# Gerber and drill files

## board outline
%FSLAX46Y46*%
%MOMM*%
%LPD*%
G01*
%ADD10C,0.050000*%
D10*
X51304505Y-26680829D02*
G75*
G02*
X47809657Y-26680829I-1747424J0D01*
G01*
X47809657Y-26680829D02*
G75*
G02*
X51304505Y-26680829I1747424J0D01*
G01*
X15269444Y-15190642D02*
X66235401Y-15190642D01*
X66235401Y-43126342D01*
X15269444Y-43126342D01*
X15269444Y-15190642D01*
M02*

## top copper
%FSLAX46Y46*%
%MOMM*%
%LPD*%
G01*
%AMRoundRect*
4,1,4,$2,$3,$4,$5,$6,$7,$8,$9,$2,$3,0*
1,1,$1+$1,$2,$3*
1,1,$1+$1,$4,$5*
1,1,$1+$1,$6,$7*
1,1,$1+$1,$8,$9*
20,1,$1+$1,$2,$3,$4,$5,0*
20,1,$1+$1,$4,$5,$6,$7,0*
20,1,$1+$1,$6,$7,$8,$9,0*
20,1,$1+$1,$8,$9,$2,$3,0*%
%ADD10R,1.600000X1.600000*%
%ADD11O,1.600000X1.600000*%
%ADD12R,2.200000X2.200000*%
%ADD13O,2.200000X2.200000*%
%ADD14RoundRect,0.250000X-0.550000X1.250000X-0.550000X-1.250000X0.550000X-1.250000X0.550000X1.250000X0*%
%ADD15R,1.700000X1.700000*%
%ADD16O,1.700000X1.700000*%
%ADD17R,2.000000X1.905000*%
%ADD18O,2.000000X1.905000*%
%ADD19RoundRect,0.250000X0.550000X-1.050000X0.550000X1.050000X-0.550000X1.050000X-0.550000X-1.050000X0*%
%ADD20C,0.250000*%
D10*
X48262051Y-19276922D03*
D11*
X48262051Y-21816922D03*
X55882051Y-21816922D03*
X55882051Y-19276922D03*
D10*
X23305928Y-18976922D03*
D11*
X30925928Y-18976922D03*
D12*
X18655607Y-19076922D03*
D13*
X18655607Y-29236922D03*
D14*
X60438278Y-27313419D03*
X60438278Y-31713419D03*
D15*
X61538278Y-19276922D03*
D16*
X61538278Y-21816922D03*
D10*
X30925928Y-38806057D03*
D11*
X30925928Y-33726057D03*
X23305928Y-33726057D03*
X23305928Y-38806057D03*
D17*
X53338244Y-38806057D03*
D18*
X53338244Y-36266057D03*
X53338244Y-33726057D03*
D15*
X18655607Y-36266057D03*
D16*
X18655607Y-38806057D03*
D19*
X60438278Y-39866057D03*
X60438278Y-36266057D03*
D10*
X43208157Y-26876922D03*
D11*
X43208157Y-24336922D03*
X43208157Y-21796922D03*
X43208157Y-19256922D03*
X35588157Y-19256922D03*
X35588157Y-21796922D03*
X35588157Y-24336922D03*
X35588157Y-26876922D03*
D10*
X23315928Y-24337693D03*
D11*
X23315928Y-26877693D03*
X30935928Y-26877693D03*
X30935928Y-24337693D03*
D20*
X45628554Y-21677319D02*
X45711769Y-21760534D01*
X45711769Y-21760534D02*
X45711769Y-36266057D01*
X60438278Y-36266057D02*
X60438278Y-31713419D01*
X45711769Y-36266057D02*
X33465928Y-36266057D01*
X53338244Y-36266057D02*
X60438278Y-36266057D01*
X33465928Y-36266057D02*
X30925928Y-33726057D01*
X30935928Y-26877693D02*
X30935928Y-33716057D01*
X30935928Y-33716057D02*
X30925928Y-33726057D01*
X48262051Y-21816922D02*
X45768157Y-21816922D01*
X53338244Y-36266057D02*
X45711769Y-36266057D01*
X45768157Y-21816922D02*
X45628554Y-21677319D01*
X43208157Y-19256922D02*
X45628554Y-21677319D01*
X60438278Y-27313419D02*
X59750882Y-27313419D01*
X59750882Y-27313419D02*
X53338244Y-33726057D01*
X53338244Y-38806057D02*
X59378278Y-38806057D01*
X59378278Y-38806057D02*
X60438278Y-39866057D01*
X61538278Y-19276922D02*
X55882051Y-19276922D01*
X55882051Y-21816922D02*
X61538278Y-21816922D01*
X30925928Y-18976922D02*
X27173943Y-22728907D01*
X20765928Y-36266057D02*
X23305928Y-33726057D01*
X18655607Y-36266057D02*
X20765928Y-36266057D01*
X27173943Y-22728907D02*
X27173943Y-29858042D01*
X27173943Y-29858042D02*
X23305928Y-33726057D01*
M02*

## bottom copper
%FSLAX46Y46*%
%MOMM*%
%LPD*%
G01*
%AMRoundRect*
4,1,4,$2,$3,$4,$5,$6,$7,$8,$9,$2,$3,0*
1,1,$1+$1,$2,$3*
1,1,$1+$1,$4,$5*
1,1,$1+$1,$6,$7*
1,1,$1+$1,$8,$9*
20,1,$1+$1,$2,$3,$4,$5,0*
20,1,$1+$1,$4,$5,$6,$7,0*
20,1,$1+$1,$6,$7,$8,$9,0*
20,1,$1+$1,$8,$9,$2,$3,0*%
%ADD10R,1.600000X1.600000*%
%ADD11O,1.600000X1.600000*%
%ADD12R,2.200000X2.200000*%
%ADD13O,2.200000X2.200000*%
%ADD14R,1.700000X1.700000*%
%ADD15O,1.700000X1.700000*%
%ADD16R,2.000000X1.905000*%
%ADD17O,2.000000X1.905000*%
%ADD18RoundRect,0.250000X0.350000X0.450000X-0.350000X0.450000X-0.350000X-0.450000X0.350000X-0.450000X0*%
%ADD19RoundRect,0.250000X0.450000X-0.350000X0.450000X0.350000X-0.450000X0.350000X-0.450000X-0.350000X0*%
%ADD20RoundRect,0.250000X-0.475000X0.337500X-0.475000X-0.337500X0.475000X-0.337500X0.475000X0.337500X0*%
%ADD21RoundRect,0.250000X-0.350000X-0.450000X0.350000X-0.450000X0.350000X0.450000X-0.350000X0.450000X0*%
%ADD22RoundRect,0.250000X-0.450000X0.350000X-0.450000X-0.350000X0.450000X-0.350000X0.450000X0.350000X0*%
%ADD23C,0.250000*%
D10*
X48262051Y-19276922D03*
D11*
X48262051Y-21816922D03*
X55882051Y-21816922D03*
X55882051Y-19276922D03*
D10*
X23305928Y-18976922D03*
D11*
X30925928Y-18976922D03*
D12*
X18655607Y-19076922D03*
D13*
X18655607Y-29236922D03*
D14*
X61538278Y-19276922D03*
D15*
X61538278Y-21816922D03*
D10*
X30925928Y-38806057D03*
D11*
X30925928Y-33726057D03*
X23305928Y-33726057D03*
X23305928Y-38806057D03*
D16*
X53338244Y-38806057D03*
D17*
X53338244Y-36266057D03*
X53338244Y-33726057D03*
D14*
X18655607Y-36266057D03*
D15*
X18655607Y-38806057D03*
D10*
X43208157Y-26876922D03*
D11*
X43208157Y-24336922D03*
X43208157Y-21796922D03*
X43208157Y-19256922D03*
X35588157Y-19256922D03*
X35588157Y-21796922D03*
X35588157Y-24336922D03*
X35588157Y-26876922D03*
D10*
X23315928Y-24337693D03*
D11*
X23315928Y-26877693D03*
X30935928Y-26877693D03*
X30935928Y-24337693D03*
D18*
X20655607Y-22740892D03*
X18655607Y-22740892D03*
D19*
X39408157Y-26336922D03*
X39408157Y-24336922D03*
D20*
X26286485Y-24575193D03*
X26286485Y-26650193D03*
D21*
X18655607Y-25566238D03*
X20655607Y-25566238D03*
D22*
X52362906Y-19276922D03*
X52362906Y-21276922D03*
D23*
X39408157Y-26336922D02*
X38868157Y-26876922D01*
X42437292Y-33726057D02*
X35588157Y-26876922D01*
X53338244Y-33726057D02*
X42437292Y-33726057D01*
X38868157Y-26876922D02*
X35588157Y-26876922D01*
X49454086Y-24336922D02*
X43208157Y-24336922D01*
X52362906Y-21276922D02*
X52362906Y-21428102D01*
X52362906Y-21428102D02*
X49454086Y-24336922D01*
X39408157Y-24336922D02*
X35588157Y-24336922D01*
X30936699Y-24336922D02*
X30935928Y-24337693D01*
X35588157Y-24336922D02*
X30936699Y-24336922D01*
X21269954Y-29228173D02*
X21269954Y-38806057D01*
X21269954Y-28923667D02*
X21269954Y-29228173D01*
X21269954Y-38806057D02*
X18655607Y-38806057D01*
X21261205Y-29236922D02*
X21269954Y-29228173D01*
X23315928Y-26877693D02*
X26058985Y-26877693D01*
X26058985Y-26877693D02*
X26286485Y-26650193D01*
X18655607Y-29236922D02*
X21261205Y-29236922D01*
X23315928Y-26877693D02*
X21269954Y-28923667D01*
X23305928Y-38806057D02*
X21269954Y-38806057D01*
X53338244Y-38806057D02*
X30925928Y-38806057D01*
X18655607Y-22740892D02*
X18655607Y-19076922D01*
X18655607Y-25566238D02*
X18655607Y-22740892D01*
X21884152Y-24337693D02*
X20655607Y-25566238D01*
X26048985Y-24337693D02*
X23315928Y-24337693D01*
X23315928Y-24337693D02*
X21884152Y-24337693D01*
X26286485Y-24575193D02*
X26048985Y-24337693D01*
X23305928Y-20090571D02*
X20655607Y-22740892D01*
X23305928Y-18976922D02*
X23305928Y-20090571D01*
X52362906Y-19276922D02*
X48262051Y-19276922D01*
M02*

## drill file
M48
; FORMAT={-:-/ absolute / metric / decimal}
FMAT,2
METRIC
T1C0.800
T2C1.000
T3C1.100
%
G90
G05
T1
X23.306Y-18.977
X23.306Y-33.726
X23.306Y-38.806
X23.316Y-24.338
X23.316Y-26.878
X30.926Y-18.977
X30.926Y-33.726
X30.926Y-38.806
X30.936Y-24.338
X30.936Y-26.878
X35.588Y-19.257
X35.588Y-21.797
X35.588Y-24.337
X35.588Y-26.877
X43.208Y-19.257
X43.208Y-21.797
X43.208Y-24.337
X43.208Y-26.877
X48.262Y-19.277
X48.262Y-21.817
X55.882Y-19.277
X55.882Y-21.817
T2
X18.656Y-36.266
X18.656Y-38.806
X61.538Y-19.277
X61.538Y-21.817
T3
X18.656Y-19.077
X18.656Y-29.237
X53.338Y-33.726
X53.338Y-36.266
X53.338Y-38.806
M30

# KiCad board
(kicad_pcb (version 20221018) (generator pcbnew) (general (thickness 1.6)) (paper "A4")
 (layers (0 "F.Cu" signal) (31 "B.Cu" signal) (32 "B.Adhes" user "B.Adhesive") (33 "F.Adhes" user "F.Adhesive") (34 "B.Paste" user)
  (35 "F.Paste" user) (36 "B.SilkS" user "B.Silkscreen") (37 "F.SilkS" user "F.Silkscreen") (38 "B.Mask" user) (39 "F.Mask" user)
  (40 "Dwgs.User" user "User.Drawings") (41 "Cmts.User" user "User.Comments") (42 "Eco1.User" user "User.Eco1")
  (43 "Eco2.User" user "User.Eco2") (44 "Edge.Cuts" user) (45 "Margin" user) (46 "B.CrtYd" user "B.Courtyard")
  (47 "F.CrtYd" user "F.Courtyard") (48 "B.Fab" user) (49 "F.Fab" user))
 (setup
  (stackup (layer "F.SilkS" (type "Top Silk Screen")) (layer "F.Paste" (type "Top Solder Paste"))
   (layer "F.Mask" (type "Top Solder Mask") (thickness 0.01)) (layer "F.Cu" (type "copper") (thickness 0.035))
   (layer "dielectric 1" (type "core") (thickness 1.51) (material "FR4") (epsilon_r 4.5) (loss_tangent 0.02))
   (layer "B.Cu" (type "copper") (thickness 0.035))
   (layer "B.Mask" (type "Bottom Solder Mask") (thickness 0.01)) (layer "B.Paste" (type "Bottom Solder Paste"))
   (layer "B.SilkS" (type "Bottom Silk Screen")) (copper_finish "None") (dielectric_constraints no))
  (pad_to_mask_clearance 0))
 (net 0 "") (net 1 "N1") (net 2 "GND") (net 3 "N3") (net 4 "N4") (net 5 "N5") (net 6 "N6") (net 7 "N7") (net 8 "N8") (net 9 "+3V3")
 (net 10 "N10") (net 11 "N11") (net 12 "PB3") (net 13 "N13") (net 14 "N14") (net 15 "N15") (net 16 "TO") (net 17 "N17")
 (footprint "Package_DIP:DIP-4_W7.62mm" (layer "F.Cu") (at 48.262051 19.276922)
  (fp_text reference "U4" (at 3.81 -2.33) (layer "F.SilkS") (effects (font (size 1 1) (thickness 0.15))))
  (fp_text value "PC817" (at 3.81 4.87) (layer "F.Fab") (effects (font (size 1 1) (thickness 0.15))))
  (pad "1" thru_hole rect (at 0 0) (size 1.6 1.6) (drill 0.8) (layers "*.Cu" "*.Mask") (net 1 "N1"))
  (pad "2" thru_hole oval (at 0 2.54) (size 1.6 1.6) (drill 0.8) (layers "*.Cu" "*.Mask") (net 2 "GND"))
  (pad "3" thru_hole oval (at 7.62 2.54) (size 1.6 1.6) (drill 0.8) (layers "*.Cu" "*.Mask") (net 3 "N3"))
  (pad "4" thru_hole oval (at 7.62 0) (size 1.6 1.6) (drill 0.8) (layers "*.Cu" "*.Mask") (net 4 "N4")))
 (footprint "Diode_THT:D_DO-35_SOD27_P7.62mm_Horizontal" (layer "F.Cu") (at 23.305928 18.976922)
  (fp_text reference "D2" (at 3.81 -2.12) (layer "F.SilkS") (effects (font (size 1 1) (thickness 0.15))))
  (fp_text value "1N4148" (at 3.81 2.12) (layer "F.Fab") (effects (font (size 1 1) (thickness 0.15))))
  (pad "1" thru_hole rect (at 0 0) (size 1.6 1.6) (drill 0.8) (layers "*.Cu" "*.Mask") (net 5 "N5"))
  (pad "2" thru_hole oval (at 7.62 0) (size 1.6 1.6) (drill 0.8) (layers "*.Cu" "*.Mask") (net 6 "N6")))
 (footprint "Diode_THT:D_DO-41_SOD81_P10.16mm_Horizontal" (layer "F.Cu") (at 18.655607 19.076922 -90)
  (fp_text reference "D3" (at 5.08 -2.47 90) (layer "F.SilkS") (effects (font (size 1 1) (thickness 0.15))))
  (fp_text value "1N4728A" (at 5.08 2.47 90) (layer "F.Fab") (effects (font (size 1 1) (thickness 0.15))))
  (pad "1" thru_hole rect (at 0 0 270) (size 2.2 2.2) (drill 1.1) (layers "*.Cu" "*.Mask") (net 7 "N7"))
  (pad "2" thru_hole oval (at 10.16 0 270) (size 2.2 2.2) (drill 1.1) (layers "*.Cu" "*.Mask") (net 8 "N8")))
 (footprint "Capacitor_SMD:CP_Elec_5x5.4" (layer "F.Cu") (at 60.438278 29.513419 -90)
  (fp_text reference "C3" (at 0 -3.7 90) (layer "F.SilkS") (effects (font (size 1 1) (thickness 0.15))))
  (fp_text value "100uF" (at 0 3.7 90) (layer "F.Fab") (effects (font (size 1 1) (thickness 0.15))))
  (pad "1" smd roundrect (at -2.2 0 270) (size 3 1.6) (layers "F.Cu" "F.Paste" "F.Mask") (roundrect_rratio 0.15625) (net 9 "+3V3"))
  (pad "2" smd roundrect (at 2.2 0 270) (size 3 1.6) (layers "F.Cu" "F.Paste" "F.Mask") (roundrect_rratio 0.15625) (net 2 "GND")))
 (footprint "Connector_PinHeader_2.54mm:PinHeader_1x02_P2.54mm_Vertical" (layer "F.Cu") (at 61.538278 19.276922)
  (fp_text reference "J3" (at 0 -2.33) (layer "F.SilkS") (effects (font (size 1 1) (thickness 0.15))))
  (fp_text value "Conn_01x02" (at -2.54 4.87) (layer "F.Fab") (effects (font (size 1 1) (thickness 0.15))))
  (pad "1" thru_hole rect (at 0 0) (size 1.7 1.7) (drill 1) (layers "*.Cu" "*.Mask") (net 4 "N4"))
  (pad "2" thru_hole oval (at 0 2.54) (size 1.7 1.7) (drill 1) (layers "*.Cu" "*.Mask") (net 3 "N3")))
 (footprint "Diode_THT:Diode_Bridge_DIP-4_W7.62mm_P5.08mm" (layer "F.Cu") (at 30.925928 38.806057 180)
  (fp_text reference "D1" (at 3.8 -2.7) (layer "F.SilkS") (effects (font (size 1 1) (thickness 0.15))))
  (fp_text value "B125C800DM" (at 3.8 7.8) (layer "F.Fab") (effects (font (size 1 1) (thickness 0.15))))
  (pad "1" thru_hole rect (at 0 0 180) (size 1.6 1.6) (drill 0.8) (layers "*.Cu" "*.Mask") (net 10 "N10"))
  (pad "2" thru_hole oval (at 0 5.08 180) (size 1.6 1.6) (drill 0.8) (layers "*.Cu" "*.Mask") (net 2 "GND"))
  (pad "3" thru_hole oval (at 7.62 5.08 180) (size 1.6 1.6) (drill 0.8) (layers "*.Cu" "*.Mask") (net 6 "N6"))
  (pad "4" thru_hole oval (at 7.62 0 180) (size 1.6 1.6) (drill 0.8) (layers "*.Cu" "*.Mask") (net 8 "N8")))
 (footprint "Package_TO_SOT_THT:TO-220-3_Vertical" (layer "F.Cu") (at 53.338244 38.806057 90)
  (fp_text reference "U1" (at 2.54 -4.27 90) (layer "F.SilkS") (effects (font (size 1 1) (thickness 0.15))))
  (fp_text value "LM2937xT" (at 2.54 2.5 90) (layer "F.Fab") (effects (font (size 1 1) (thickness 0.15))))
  (pad "1" thru_hole rect (at 0 0 90) (size 1.905 2) (drill 1.1) (layers "*.Cu" "*.Mask") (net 10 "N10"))
  (pad "2" thru_hole oval (at 2.54 0 90) (size 1.905 2) (drill 1.1) (layers "*.Cu" "*.Mask") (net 2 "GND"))
  (pad "3" thru_hole oval (at 5.08 0 90) (size 1.905 2) (drill 1.1) (layers "*.Cu" "*.Mask") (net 9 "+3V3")))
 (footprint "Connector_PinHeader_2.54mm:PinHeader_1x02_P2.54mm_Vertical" (layer "F.Cu") (at 18.655607 36.266057)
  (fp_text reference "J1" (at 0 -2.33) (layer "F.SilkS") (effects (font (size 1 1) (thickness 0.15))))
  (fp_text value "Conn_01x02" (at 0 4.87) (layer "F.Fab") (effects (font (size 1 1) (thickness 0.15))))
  (pad "1" thru_hole rect (at 0 0) (size 1.7 1.7) (drill 1) (layers "*.Cu" "*.Mask") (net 6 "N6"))
  (pad "2" thru_hole oval (at 0 2.54) (size 1.7 1.7) (drill 1) (layers "*.Cu" "*.Mask") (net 8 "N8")))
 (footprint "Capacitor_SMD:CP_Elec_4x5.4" (layer "F.Cu") (at 60.438278 38.066057 90)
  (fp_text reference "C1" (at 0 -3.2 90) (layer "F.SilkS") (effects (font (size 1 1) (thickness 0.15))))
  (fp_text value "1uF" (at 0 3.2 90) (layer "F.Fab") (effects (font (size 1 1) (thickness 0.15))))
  (pad "1" smd roundrect (at -1.8 0 90) (size 2.6 1.6) (layers "F.Cu" "F.Paste" "F.Mask") (roundrect_rratio 0.15625) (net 10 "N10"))
  (pad "2" smd roundrect (at 1.8 0 90) (size 2.6 1.6) (layers "F.Cu" "F.Paste" "F.Mask") (roundrect_rratio 0.15625) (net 2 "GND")))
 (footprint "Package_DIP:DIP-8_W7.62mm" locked (layer "F.Cu") (at 43.208157 26.876922 180)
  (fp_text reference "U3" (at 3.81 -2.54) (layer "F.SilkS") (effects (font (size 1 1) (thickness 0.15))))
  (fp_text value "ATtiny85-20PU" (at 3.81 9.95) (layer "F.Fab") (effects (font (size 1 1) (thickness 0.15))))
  (pad "1" thru_hole rect locked (at 0 0 180) (size 1.6 1.6) (drill 0.8) (layers "*.Cu" "*.Mask") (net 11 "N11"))
  (pad "2" thru_hole oval locked (at 0 2.54 180) (size 1.6 1.6) (drill 0.8) (layers "*.Cu" "*.Mask") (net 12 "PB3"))
  (pad "3" thru_hole oval locked (at 0 5.08 180) (size 1.6 1.6) (drill 0.8) (layers "*.Cu" "*.Mask") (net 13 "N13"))
  (pad "4" thru_hole oval locked (at 0 7.62 180) (size 1.6 1.6) (drill 0.8) (layers "*.Cu" "*.Mask") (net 2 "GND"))
  (pad "5" thru_hole oval locked (at 7.62 7.62 180) (size 1.6 1.6) (drill 0.8) (layers "*.Cu" "*.Mask") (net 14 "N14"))
  (pad "6" thru_hole oval locked (at 7.62 5.08 180) (size 1.6 1.6) (drill 0.8) (layers "*.Cu" "*.Mask") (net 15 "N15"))
  (pad "7" thru_hole oval locked (at 7.62 2.54 180) (size 1.6 1.6) (drill 0.8) (layers "*.Cu" "*.Mask") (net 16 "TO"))
  (pad "8" thru_hole oval locked (at 7.62 0 180) (size 1.6 1.6) (drill 0.8) (layers "*.Cu" "*.Mask") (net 9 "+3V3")))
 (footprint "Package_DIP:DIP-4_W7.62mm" (layer "F.Cu") (at 23.315928 24.337693)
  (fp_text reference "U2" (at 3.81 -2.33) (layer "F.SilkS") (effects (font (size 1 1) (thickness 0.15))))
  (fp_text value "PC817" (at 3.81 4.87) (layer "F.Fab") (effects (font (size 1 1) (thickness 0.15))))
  (pad "1" thru_hole rect (at 0 0) (size 1.6 1.6) (drill 0.8) (layers "*.Cu" "*.Mask") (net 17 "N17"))
  (pad "2" thru_hole oval (at 0 2.54) (size 1.6 1.6) (drill 0.8) (layers "*.Cu" "*.Mask") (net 8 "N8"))
  (pad "3" thru_hole oval (at 7.62 2.54) (size 1.6 1.6) (drill 0.8) (layers "*.Cu" "*.Mask") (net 2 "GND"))
  (pad "4" thru_hole oval (at 7.62 0) (size 1.6 1.6) (drill 0.8) (layers "*.Cu" "*.Mask") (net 16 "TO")))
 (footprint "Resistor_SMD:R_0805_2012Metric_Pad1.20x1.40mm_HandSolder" (layer "B.Cu") (at 19.655607 22.740892 180)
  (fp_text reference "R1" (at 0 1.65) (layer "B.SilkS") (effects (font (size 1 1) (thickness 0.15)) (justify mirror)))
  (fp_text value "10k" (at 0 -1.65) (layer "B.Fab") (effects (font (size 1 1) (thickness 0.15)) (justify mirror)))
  (pad "1" smd roundrect (at -1 0 180) (size 1.2 1.4) (layers "B.Cu" "B.Paste" "B.Mask") (roundrect_rratio 0.208333) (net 5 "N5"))
  (pad "2" smd roundrect (at 1 0 180) (size 1.2 1.4) (layers "B.Cu" "B.Paste" "B.Mask") (roundrect_rratio 0.208333) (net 7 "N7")))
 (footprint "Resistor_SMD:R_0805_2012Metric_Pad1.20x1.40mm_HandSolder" (layer "B.Cu") (at 39.408157 25.336922 90)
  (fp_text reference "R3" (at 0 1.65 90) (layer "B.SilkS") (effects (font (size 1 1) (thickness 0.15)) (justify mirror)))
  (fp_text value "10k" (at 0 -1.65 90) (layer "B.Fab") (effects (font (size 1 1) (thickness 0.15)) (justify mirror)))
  (pad "1" smd roundrect (at -1 0 90) (size 1.2 1.4) (layers "B.Cu" "B.Paste" "B.Mask") (roundrect_rratio 0.208333) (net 9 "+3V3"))
  (pad "2" smd roundrect (at 1 0 90) (size 1.2 1.4) (layers "B.Cu" "B.Paste" "B.Mask") (roundrect_rratio 0.208333) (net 16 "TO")))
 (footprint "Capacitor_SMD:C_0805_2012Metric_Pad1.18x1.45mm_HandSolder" (layer "B.Cu") (at 26.286485 25.612693 -90)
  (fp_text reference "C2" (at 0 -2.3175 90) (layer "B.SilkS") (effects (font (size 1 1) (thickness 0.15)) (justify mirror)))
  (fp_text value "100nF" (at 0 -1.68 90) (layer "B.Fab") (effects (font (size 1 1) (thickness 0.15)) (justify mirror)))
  (pad "1" smd roundrect (at -1.0375 0 270) (size 1.175 1.45) (layers "B.Cu" "B.Paste" "B.Mask") (roundrect_rratio 0.212766) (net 17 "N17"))
  (pad "2" smd roundrect (at 1.0375 0 270) (size 1.175 1.45) (layers "B.Cu" "B.Paste" "B.Mask") (roundrect_rratio 0.212766) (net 8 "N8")))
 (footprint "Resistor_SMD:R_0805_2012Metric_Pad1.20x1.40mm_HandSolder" (layer "B.Cu") (at 19.655607 25.566238)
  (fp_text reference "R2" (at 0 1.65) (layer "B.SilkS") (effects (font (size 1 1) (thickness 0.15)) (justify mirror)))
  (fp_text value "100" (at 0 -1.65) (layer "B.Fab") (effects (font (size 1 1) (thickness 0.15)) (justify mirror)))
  (pad "1" smd roundrect (at -1 0) (size 1.2 1.4) (layers "B.Cu" "B.Paste" "B.Mask") (roundrect_rratio 0.208333) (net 7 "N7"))
  (pad "2" smd roundrect (at 1 0) (size 1.2 1.4) (layers "B.Cu" "B.Paste" "B.Mask") (roundrect_rratio 0.208333) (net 17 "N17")))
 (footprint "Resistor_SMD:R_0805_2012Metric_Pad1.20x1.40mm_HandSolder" (layer "B.Cu") (at 52.362906 20.276922 -90)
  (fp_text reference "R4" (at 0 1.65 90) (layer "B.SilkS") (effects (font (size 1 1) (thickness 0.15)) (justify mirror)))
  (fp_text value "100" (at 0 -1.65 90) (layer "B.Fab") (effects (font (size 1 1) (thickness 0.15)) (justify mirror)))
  (pad "1" smd roundrect (at -1 0 270) (size 1.2 1.4) (layers "B.Cu" "B.Paste" "B.Mask") (roundrect_rratio 0.208333) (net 1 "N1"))
  (pad "2" smd roundrect (at 1 0 270) (size 1.2 1.4) (layers "B.Cu" "B.Paste" "B.Mask") (roundrect_rratio 0.208333) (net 12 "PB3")))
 (gr_circle (center 49.557081 26.680829) (end 50.875697 27.827451) (stroke (width 0.05) (type default)) (fill none) (layer "Edge.Cuts"))
 (gr_rect (start 15.269444 15.190642) (end 66.235401 43.126342) (stroke (width 0.05) (type default)) (fill none) (layer "Edge.Cuts"))
 (segment (start 45.628554 21.677319) (end 45.711769 21.760534) (width 0.25) (layer "F.Cu") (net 2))
 (segment (start 45.711769 21.760534) (end 45.711769 36.266057) (width 0.25) (layer "F.Cu") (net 2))
 (segment (start 60.438278 36.266057) (end 60.438278 31.713419) (width 0.25) (layer "F.Cu") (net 2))
 (segment (start 45.711769 36.266057) (end 33.465928 36.266057) (width 0.25) (layer "F.Cu") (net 2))
 (segment (start 53.338244 36.266057) (end 60.438278 36.266057) (width 0.25) (layer "F.Cu") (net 2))
 (segment (start 33.465928 36.266057) (end 30.925928 33.726057) (width 0.25) (layer "F.Cu") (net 2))
 (segment (start 30.935928 26.877693) (end 30.935928 33.716057) (width 0.25) (layer "F.Cu") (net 2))
 (segment (start 30.935928 33.716057) (end 30.925928 33.726057) (width 0.25) (layer "F.Cu") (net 2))
 (segment (start 48.262051 21.816922) (end 45.768157 21.816922) (width 0.25) (layer "F.Cu") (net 2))
 (segment (start 53.338244 36.266057) (end 45.711769 36.266057) (width 0.25) (layer "F.Cu") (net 2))
 (segment (start 45.768157 21.816922) (end 45.628554 21.677319) (width 0.25) (layer "F.Cu") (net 2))
 (segment (start 43.208157 19.256922) (end 45.628554 21.677319) (width 0.25) (layer "F.Cu") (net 2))
 (segment (start 60.438278 27.313419) (end 59.750882 27.313419) (width 0.25) (layer "F.Cu") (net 9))
 (segment (start 59.750882 27.313419) (end 53.338244 33.726057) (width 0.25) (layer "F.Cu") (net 9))
 (segment (start 39.408157 26.336922) (end 38.868157 26.876922) (width 0.25) (layer "B.Cu") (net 9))
 (segment (start 42.437292 33.726057) (end 35.588157 26.876922) (width 0.25) (layer "B.Cu") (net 9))
 (segment (start 53.338244 33.726057) (end 42.437292 33.726057) (width 0.25) (layer "B.Cu") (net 9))
 (segment (start 38.868157 26.876922) (end 35.588157 26.876922) (width 0.25) (layer "B.Cu") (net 9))
 (segment (start 49.454086 24.336922) (end 43.208157 24.336922) (width 0.25) (layer "B.Cu") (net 12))
 (segment (start 52.362906 21.276922) (end 52.362906 21.428102) (width 0.25) (layer "B.Cu") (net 12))
 (segment (start 52.362906 21.428102) (end 49.454086 24.336922) (width 0.25) (layer "B.Cu") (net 12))
 (segment (start 39.408157 24.336922) (end 35.588157 24.336922) (width 0.25) (layer "B.Cu") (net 16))
 (segment (start 30.936699 24.336922) (end 30.935928 24.337693) (width 0.25) (layer "B.Cu") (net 16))
 (segment (start 35.588157 24.336922) (end 30.936699 24.336922) (width 0.25) (layer "B.Cu") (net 16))
 (segment (start 21.269954 29.228173) (end 21.269954 38.806057) (width 0.25) (layer "B.Cu") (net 8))
 (segment (start 21.269954 28.923667) (end 21.269954 29.228173) (width 0.25) (layer "B.Cu") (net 8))
 (segment (start 21.269954 38.806057) (end 18.655607 38.806057) (width 0.25) (layer "B.Cu") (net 8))
 (segment (start 21.261205 29.236922) (end 21.269954 29.228173) (width 0.25) (layer "B.Cu") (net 8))
 (segment (start 23.315928 26.877693) (end 26.058985 26.877693) (width 0.25) (layer "B.Cu") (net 8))
 (segment (start 26.058985 26.877693) (end 26.286485 26.650193) (width 0.25) (layer "B.Cu") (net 8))
 (segment (start 18.655607 29.236922) (end 21.261205 29.236922) (width 0.25) (layer "B.Cu") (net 8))
 (segment (start 23.315928 26.877693) (end 21.269954 28.923667) (width 0.25) (layer "B.Cu") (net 8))
 (segment (start 23.305928 38.806057) (end 21.269954 38.806057) (width 0.25) (layer "B.Cu") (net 8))
 (segment (start 53.338244 38.806057) (end 59.378278 38.806057) (width 0.25) (layer "F.Cu") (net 10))
 (segment (start 59.378278 38.806057) (end 60.438278 39.866057) (width 0.25) (layer "F.Cu") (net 10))
 (segment (start 53.338244 38.806057) (end 30.925928 38.806057) (width 0.25) (layer "B.Cu") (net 10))
 (segment (start 18.655607 22.740892) (end 18.655607 19.076922) (width 0.25) (layer "B.Cu") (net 7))
 (segment (start 18.655607 25.566238) (end 18.655607 22.740892) (width 0.25) (layer "B.Cu") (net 7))
 (segment (start 61.538278 19.276922) (end 55.882051 19.276922) (width 0.25) (layer "F.Cu") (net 4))
 (segment (start 55.882051 21.816922) (end 61.538278 21.816922) (width 0.25) (layer "F.Cu") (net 3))
 (segment (start 21.884152 24.337693) (end 20.655607 25.566238) (width 0.25) (layer "B.Cu") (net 17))
 (segment (start 26.048985 24.337693) (end 23.315928 24.337693) (width 0.25) (layer "B.Cu") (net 17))
 (segment (start 23.315928 24.337693) (end 21.884152 24.337693) (width 0.25) (layer "B.Cu") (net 17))
 (segment (start 26.286485 24.575193) (end 26.048985 24.337693) (width 0.25) (layer "B.Cu") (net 17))
 (segment (start 30.925928 18.976922) (end 27.173943 22.728907) (width 0.25) (layer "F.Cu") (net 6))
 (segment (start 20.765928 36.266057) (end 23.305928 33.726057) (width 0.25) (layer "F.Cu") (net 6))
 (segment (start 18.655607 36.266057) (end 20.765928 36.266057) (width 0.25) (layer "F.Cu") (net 6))
 (segment (start 27.173943 22.728907) (end 27.173943 29.858042) (width 0.25) (layer "F.Cu") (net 6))
 (segment (start 27.173943 29.858042) (end 23.305928 33.726057) (width 0.25) (layer "F.Cu") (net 6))
 (segment (start 23.305928 20.090571) (end 20.655607 22.740892) (width 0.25) (layer "B.Cu") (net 5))
 (segment (start 23.305928 18.976922) (end 23.305928 20.090571) (width 0.25) (layer "B.Cu") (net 5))
 (segment (start 52.362906 19.276922) (end 48.262051 19.276922) (width 0.25) (layer "B.Cu") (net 1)))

